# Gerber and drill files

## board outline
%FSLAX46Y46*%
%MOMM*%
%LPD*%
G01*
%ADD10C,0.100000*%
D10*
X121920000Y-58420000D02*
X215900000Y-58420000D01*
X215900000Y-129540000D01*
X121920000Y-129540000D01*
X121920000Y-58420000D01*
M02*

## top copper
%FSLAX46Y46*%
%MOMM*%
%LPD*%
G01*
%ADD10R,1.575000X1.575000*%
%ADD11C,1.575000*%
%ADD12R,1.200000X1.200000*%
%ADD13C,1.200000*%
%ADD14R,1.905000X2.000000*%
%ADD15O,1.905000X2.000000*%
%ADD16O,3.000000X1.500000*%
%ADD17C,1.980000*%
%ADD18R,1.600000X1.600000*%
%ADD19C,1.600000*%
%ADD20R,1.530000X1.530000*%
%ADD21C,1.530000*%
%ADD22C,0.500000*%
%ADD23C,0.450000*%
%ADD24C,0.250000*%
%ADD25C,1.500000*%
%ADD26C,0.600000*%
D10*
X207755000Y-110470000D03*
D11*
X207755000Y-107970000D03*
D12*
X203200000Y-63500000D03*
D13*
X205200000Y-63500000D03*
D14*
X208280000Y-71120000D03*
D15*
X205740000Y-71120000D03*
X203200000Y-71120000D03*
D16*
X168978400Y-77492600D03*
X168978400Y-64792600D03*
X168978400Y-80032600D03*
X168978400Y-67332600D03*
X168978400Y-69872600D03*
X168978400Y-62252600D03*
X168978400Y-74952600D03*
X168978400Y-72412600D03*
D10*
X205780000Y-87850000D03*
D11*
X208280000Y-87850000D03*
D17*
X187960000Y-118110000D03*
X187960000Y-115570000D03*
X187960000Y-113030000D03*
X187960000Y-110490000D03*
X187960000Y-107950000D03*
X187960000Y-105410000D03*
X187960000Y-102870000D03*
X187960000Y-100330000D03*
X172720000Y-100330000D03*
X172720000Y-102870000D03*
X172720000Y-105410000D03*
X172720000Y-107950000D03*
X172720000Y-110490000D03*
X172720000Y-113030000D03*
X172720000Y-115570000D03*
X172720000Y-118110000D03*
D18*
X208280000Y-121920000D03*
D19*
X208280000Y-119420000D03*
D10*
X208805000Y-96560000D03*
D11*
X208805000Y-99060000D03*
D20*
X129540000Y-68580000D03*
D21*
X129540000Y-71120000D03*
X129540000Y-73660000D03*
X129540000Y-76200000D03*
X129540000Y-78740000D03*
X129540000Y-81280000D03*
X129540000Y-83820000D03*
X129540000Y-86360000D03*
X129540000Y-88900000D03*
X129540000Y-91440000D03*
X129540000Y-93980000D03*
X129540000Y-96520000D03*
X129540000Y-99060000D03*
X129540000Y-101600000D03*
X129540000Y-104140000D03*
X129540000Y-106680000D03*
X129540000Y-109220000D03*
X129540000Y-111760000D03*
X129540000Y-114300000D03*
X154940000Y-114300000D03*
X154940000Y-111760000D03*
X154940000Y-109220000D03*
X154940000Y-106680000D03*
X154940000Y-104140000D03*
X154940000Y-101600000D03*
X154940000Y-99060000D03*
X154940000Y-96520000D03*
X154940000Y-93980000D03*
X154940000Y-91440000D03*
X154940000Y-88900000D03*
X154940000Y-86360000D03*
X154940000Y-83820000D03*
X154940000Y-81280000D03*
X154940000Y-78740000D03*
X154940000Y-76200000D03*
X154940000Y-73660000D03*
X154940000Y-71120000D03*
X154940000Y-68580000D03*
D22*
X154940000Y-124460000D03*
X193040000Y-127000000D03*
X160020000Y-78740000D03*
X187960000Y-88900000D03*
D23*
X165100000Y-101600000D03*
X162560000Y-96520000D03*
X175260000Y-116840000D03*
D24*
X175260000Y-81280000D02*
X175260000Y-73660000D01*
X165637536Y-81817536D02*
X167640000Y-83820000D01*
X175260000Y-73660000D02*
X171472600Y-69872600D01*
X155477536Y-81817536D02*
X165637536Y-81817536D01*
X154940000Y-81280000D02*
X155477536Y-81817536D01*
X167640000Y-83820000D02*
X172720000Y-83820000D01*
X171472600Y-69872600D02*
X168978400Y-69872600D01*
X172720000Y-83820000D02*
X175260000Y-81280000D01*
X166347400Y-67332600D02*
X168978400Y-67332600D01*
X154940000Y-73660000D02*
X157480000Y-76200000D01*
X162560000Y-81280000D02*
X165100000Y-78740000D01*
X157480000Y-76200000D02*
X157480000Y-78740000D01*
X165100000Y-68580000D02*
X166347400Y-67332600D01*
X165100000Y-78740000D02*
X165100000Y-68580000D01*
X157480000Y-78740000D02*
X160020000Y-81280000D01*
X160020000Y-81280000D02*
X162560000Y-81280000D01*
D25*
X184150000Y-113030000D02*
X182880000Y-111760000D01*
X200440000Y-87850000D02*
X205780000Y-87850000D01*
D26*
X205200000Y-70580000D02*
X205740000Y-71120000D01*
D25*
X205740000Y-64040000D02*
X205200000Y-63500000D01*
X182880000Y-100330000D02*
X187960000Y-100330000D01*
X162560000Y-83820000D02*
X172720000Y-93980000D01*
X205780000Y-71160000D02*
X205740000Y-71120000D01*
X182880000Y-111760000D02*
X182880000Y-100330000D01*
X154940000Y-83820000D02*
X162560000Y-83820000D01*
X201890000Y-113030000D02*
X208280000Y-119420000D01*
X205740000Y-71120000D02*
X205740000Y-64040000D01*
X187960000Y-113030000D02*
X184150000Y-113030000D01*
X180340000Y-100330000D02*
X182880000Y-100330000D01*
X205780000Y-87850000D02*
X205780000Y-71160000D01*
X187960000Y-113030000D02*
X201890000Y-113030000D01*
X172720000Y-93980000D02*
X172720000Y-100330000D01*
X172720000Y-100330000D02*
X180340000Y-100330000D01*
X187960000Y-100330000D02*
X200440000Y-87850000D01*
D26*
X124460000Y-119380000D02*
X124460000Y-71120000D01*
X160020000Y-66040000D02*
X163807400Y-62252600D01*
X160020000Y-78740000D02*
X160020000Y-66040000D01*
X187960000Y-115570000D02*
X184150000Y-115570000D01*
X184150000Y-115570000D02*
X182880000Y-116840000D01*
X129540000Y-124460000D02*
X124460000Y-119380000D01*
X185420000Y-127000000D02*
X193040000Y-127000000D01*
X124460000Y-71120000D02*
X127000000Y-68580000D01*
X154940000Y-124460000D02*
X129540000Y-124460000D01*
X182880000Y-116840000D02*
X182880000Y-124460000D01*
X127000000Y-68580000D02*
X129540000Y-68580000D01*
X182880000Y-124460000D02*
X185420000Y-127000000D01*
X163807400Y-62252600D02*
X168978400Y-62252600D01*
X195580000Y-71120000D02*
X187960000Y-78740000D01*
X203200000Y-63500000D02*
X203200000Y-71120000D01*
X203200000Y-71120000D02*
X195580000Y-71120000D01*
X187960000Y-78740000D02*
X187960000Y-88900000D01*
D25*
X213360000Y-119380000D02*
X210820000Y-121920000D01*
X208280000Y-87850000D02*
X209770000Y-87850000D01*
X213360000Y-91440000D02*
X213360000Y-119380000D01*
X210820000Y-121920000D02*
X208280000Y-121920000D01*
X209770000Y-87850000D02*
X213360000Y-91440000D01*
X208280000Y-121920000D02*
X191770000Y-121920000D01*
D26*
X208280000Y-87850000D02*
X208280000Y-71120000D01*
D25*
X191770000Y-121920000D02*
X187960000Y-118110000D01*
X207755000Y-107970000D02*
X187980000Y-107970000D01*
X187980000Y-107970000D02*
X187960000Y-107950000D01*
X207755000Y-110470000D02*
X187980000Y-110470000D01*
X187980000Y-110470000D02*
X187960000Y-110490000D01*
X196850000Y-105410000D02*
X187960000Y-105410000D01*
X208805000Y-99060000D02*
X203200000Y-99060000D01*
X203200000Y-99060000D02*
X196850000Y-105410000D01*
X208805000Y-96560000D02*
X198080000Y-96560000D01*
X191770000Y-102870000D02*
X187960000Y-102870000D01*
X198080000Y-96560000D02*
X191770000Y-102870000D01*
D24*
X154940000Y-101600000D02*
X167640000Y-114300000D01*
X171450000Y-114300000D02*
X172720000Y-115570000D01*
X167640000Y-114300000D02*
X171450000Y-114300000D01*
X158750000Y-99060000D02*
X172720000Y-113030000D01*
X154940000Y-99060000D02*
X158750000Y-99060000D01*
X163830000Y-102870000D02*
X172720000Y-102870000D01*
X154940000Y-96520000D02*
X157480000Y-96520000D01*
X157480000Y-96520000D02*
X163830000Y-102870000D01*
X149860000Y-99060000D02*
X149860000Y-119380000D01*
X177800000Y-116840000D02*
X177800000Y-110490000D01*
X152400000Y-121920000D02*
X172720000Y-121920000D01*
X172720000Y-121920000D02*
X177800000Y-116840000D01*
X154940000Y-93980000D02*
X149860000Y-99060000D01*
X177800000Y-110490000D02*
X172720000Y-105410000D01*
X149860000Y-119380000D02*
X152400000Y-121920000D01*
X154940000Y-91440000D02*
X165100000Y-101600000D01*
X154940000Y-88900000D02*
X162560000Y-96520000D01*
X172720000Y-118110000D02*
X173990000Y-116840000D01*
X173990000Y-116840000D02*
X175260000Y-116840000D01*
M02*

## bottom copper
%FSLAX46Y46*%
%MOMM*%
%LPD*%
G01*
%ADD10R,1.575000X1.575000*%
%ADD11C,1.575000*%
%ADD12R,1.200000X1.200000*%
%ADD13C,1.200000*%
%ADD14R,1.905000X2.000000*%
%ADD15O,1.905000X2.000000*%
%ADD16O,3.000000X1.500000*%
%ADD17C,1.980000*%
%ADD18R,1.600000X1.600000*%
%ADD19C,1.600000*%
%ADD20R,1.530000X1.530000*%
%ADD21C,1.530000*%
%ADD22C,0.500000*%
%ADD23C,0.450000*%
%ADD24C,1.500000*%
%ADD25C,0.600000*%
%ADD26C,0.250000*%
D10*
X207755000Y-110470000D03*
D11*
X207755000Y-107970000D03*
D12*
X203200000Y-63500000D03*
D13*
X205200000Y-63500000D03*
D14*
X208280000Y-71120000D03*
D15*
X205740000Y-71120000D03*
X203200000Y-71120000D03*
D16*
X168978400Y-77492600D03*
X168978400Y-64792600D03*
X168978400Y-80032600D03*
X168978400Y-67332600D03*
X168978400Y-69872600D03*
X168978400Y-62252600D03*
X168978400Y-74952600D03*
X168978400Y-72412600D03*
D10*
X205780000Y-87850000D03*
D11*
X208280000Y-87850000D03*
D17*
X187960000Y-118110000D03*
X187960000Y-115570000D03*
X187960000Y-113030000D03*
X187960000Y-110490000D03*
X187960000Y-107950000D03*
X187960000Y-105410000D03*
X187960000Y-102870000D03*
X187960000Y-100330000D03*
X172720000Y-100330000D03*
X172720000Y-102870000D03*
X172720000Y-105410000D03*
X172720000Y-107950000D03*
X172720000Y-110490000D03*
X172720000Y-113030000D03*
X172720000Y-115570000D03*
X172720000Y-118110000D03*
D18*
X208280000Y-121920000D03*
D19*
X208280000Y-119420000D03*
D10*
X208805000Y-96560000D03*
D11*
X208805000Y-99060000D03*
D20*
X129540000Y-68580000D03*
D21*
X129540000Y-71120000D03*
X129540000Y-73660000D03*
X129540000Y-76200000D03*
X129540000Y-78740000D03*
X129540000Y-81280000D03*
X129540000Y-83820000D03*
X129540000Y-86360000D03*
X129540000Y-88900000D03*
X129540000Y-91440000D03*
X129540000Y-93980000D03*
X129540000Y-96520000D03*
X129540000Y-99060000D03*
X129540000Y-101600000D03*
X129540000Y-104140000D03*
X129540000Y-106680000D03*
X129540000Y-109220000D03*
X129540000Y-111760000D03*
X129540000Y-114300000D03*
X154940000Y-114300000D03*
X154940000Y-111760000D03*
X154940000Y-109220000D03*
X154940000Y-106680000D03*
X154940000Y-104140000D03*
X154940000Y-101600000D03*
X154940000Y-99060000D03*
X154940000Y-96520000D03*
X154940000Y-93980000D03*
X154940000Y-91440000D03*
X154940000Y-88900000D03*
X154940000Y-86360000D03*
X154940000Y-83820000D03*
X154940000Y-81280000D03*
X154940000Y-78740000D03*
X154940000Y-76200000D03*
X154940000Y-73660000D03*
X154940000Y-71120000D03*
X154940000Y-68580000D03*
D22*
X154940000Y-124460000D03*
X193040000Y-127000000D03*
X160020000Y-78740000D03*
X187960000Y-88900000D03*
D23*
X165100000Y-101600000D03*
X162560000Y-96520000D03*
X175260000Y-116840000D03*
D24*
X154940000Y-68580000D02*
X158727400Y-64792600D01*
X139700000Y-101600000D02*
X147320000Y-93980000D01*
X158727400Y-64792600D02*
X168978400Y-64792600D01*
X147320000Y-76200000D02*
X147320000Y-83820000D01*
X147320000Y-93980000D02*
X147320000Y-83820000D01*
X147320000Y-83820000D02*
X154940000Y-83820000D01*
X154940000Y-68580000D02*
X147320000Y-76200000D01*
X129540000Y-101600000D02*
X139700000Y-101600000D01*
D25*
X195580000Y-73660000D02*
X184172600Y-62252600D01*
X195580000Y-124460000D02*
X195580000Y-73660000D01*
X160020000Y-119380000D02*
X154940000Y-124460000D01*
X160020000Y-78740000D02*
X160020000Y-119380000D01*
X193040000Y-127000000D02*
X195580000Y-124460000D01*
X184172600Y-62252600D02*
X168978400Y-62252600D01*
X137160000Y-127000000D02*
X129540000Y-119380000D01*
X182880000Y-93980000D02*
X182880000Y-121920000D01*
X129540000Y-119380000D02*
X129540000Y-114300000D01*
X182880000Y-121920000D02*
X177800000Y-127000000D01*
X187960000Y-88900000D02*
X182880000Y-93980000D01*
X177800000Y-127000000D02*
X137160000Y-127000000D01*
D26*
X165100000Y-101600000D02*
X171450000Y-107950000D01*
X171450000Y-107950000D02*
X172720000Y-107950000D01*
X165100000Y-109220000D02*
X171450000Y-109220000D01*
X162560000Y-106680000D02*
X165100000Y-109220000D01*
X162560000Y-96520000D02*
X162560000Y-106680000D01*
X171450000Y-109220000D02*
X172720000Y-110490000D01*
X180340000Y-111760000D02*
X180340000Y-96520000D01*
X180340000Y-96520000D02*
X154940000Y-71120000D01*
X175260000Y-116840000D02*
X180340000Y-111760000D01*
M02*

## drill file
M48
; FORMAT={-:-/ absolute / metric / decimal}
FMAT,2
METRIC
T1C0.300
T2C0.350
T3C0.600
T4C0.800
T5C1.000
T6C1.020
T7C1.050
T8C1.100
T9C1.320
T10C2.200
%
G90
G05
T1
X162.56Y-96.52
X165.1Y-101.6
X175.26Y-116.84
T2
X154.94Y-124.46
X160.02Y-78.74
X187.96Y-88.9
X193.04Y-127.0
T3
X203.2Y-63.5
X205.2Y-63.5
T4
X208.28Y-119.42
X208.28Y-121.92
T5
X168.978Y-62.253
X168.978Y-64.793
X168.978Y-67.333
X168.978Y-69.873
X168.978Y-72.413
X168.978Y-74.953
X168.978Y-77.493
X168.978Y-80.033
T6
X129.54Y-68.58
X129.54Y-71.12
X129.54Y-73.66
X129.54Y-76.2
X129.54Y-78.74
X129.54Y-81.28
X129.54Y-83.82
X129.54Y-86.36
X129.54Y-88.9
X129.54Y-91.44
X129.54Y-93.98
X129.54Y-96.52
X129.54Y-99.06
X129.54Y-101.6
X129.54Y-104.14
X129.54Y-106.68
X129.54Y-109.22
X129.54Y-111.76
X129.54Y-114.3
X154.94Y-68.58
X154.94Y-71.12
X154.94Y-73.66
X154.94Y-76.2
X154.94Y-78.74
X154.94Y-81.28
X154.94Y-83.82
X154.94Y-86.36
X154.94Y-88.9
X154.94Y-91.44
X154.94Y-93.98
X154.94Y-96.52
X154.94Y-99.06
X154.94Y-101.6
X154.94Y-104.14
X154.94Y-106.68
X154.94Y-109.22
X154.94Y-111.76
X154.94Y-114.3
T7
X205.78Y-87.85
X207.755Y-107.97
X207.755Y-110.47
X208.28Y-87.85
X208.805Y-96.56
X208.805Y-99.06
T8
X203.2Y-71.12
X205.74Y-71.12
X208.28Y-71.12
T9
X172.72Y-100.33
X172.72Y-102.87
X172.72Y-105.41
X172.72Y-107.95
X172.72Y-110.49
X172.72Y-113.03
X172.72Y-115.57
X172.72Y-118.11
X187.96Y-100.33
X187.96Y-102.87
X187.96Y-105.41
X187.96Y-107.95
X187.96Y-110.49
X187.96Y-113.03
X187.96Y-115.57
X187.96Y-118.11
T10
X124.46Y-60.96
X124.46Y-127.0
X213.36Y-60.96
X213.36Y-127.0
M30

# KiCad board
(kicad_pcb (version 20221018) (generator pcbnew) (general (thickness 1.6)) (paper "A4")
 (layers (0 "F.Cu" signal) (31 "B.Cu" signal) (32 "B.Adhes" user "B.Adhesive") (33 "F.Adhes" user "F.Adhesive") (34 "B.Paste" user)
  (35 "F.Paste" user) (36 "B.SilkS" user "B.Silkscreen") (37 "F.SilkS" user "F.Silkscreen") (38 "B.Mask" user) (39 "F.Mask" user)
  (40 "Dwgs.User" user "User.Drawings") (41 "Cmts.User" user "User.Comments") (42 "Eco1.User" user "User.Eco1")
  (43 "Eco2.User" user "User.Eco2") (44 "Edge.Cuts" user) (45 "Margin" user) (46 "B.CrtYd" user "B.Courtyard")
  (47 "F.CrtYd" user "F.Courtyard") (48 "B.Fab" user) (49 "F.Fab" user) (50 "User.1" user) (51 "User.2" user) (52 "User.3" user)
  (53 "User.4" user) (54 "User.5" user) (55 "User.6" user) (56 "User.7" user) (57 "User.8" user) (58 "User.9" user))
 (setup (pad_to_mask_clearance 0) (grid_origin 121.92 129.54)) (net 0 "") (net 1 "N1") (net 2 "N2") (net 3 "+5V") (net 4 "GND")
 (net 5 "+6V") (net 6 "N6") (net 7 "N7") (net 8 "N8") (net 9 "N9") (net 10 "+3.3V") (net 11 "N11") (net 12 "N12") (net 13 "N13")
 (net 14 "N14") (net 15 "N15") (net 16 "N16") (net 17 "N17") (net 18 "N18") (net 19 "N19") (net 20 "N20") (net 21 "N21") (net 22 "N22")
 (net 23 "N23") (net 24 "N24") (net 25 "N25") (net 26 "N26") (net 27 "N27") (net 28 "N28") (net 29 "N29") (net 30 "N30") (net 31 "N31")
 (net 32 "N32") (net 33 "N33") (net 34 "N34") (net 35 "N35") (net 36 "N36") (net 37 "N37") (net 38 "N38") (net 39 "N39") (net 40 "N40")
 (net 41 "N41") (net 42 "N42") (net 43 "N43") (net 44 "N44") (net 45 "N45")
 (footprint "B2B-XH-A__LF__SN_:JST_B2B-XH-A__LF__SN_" (layer "F.Cu") (at 208.28 109.22 -90)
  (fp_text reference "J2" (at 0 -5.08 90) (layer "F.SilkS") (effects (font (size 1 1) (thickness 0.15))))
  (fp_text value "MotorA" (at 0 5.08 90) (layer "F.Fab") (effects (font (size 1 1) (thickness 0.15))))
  (pad "1" thru_hole rect (at 1.25 0.525 270) (size 1.575 1.575) (drill 1.05) (layers "*.Cu" "*.Mask") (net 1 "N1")
   (solder_mask_margin 0.102))
  (pad "2" thru_hole circle (at -1.25 0.525 270) (size 1.575 1.575) (drill 1.05) (layers "*.Cu" "*.Mask") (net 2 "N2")
   (solder_mask_margin 0.102)))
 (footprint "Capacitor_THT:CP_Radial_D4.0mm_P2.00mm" (layer "F.Cu") (at 203.2 63.5)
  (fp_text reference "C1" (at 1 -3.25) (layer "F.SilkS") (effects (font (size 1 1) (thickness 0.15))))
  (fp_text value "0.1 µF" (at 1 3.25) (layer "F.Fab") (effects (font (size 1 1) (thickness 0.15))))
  (pad "1" thru_hole rect (at 0 0) (size 1.2 1.2) (drill 0.6) (layers "*.Cu" "*.Mask") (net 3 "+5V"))
  (pad "2" thru_hole circle (at 2 0) (size 1.2 1.2) (drill 0.6) (layers "*.Cu" "*.Mask") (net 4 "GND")))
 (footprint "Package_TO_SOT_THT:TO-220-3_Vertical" (layer "F.Cu") (at 208.28 71.12 180)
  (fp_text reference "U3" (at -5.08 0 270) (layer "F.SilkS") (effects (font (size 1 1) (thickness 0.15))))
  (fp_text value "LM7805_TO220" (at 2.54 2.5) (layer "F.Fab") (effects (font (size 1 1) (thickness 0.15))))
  (pad "1" thru_hole rect (at 0 0 180) (size 1.905 2) (drill 1.1) (layers "*.Cu" "*.Mask") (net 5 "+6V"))
  (pad "2" thru_hole oval (at 2.54 0 180) (size 1.905 2) (drill 1.1) (layers "*.Cu" "*.Mask") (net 4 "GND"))
  (pad "3" thru_hole oval (at 5.08 0 180) (size 1.905 2) (drill 1.1) (layers "*.Cu" "*.Mask") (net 3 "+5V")))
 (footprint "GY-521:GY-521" (layer "F.Cu") (at 167.2084 82.0966)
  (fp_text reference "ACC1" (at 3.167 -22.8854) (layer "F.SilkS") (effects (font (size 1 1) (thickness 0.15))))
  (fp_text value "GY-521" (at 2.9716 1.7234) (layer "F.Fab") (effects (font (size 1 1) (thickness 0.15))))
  (pad "AD0" thru_hole oval (at 1.77 -4.604) (size 3 1.5) (drill 1) (layers "*.Cu" "*.Mask") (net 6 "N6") (solder_mask_margin 0.102))
  (pad "GND" thru_hole oval (at 1.77 -17.304) (size 3 1.5) (drill 1) (layers "*.Cu" "*.Mask") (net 4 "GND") (solder_mask_margin 0.102))
  (pad "INT" thru_hole oval (at 1.77 -2.064) (size 3 1.5) (drill 1) (layers "*.Cu" "*.Mask") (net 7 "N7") (solder_mask_margin 0.102))
  (pad "SCL" thru_hole oval (at 1.77 -14.764) (size 3 1.5) (drill 1) (layers "*.Cu" "*.Mask") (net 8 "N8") (solder_mask_margin 0.102))
  (pad "SDA" thru_hole oval (at 1.77 -12.224) (size 3 1.5) (drill 1) (layers "*.Cu" "*.Mask") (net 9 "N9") (solder_mask_margin 0.102))
  (pad "VCC" thru_hole oval (at 1.77 -19.844) (size 3 1.5) (drill 1) (layers "*.Cu" "*.Mask") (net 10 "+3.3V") (solder_mask_margin 0.102))
  (pad "XCL" thru_hole oval (at 1.77 -7.144) (size 3 1.5) (drill 1) (layers "*.Cu" "*.Mask") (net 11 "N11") (solder_mask_margin 0.102))
  (pad "XDA" thru_hole oval (at 1.77 -9.684) (size 3 1.5) (drill 1) (layers "*.Cu" "*.Mask") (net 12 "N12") (solder_mask_margin 0.102)))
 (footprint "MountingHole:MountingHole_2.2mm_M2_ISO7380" (layer "F.Cu") (at 213.36 127)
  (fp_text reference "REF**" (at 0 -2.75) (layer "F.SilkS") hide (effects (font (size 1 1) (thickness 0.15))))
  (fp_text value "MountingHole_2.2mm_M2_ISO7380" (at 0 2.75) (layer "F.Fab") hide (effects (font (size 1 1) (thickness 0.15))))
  (pad "" np_thru_hole circle (at 0 0) (size 2.2 2.2) (drill 2.2) (layers "F&B.Cu" "*.Mask")))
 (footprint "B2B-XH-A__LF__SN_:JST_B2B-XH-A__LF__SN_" (layer "F.Cu") (at 207.03 88.375 180)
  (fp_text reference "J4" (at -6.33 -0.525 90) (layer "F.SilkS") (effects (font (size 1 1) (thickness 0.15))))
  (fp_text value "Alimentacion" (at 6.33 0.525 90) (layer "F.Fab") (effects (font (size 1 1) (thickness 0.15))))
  (pad "1" thru_hole rect (at 1.25 0.525 180) (size 1.575 1.575) (drill 1.05) (layers "*.Cu" "*.Mask") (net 4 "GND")
   (solder_mask_margin 0.102))
  (pad "2" thru_hole circle (at -1.25 0.525 180) (size 1.575 1.575) (drill 1.05) (layers "*.Cu" "*.Mask") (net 5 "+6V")
   (solder_mask_margin 0.102)))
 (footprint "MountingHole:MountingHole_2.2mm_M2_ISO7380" (layer "F.Cu") (at 213.36 60.96)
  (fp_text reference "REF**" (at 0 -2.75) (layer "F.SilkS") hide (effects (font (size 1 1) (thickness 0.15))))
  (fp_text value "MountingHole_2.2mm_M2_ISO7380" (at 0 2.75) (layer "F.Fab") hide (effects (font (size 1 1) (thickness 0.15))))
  (pad "" np_thru_hole circle (at 0 0) (size 2.2 2.2) (drill 2.2) (layers "F&B.Cu" "*.Mask")))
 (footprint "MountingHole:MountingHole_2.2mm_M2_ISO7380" (layer "F.Cu") (at 124.46 60.96)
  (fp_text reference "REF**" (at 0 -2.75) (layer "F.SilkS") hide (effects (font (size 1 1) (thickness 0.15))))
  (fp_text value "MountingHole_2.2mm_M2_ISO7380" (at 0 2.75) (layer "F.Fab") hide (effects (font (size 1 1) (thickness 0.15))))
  (pad "" np_thru_hole circle (at 0 0) (size 2.2 2.2) (drill 2.2) (layers "F&B.Cu" "*.Mask")))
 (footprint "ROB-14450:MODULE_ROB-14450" (layer "F.Cu") (at 180.34 109.22 180)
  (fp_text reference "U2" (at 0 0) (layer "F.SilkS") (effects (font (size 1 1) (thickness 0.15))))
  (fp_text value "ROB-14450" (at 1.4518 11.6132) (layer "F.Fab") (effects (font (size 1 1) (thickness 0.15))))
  (pad "1" thru_hole circle (at -7.62 -8.89 180) (size 1.98 1.98) (drill 1.32) (layers "*.Cu" "*.Mask") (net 5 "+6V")
   (solder_mask_margin 0.102))
  (pad "2" thru_hole circle (at -7.62 -6.35 180) (size 1.98 1.98) (drill 1.32) (layers "*.Cu" "*.Mask") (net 10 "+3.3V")
   (solder_mask_margin 0.102))
  (pad "3" thru_hole circle (at -7.62 -3.81 180) (size 1.98 1.98) (drill 1.32) (layers "*.Cu" "*.Mask") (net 4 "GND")
   (solder_mask_margin 0.102))
  (pad "4" thru_hole circle (at -7.62 -1.27 180) (size 1.98 1.98) (drill 1.32) (layers "*.Cu" "*.Mask") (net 1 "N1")
   (solder_mask_margin 0.102))
  (pad "5" thru_hole circle (at -7.62 1.27 180) (size 1.98 1.98) (drill 1.32) (layers "*.Cu" "*.Mask") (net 2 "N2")
   (solder_mask_margin 0.102))
  (pad "6" thru_hole circle (at -7.62 3.81 180) (size 1.98 1.98) (drill 1.32) (layers "*.Cu" "*.Mask") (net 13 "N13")
   (solder_mask_margin 0.102))
  (pad "7" thru_hole circle (at -7.62 6.35 180) (size 1.98 1.98) (drill 1.32) (layers "*.Cu" "*.Mask") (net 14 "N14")
   (solder_mask_margin 0.102))
  (pad "8" thru_hole circle (at -7.62 8.89 180) (size 1.98 1.98) (drill 1.32) (layers "*.Cu" "*.Mask") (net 4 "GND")
   (solder_mask_margin 0.102))
  (pad "9" thru_hole circle (at 7.62 8.89 180) (size 1.98 1.98) (drill 1.32) (layers "*.Cu" "*.Mask") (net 4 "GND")
   (solder_mask_margin 0.102))
  (pad "10" thru_hole circle (at 7.62 6.35 180) (size 1.98 1.98) (drill 1.32) (layers "*.Cu" "*.Mask") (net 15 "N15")
   (solder_mask_margin 0.102))
  (pad "11" thru_hole circle (at 7.62 3.81 180) (size 1.98 1.98) (drill 1.32) (layers "*.Cu" "*.Mask") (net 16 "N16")
   (solder_mask_margin 0.102))
  (pad "12" thru_hole circle (at 7.62 1.27 180) (size 1.98 1.98) (drill 1.32) (layers "*.Cu" "*.Mask") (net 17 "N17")
   (solder_mask_margin 0.102))
  (pad "13" thru_hole circle (at 7.62 -1.27 180) (size 1.98 1.98) (drill 1.32) (layers "*.Cu" "*.Mask") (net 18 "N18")
   (solder_mask_margin 0.102))
  (pad "14" thru_hole circle (at 7.62 -3.81 180) (size 1.98 1.98) (drill 1.32) (layers "*.Cu" "*.Mask") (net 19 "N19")
   (solder_mask_margin 0.102))
  (pad "15" thru_hole circle (at 7.62 -6.35 180) (size 1.98 1.98) (drill 1.32) (layers "*.Cu" "*.Mask") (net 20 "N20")
   (solder_mask_margin 0.102))
  (pad "16" thru_hole circle (at 7.62 -8.89 180) (size 1.98 1.98) (drill 1.32) (layers "*.Cu" "*.Mask") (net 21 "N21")
   (solder_mask_margin 0.102)))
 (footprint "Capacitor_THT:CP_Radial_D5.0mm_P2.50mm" (layer "F.Cu") (at 208.28 121.92 90)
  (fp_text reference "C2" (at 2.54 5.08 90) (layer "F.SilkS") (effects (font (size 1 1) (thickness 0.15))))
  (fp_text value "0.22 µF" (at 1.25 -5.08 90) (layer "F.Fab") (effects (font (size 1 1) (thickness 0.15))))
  (pad "1" thru_hole rect (at 0 0 90) (size 1.6 1.6) (drill 0.8) (layers "*.Cu" "*.Mask") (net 5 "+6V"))
  (pad "2" thru_hole circle (at 2.5 0 90) (size 1.6 1.6) (drill 0.8) (layers "*.Cu" "*.Mask") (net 4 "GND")))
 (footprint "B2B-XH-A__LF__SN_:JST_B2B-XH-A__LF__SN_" (layer "F.Cu") (at 208.28 97.81 90)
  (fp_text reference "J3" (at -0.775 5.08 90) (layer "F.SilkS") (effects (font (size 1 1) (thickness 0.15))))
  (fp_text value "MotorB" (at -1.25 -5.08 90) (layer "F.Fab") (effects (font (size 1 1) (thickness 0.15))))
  (pad "1" thru_hole rect (at 1.25 0.525 90) (size 1.575 1.575) (drill 1.05) (layers "*.Cu" "*.Mask") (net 14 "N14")
   (solder_mask_margin 0.102))
  (pad "2" thru_hole circle (at -1.25 0.525 90) (size 1.575 1.575) (drill 1.05) (layers "*.Cu" "*.Mask") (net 13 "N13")
   (solder_mask_margin 0.102)))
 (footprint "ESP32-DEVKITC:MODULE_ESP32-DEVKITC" (layer "F.Cu") (at 142.24 91.43)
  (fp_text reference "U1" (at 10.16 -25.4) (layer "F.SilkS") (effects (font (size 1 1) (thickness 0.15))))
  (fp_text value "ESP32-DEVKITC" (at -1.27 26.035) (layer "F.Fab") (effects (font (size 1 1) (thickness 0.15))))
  (pad "1" thru_hole rect (at -12.7 -22.85) (size 1.53 1.53) (drill 1.02) (layers "*.Cu" "*.Mask") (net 10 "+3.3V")
   (solder_mask_margin 0.102))
  (pad "2" thru_hole circle (at -12.7 -20.31) (size 1.53 1.53) (drill 1.02) (layers "*.Cu" "*.Mask") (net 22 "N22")
   (solder_mask_margin 0.102))
  (pad "3" thru_hole circle (at -12.7 -17.77) (size 1.53 1.53) (drill 1.02) (layers "*.Cu" "*.Mask") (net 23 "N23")
   (solder_mask_margin 0.102))
  (pad "4" thru_hole circle (at -12.7 -15.23) (size 1.53 1.53) (drill 1.02) (layers "*.Cu" "*.Mask") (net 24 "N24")
   (solder_mask_margin 0.102))
  (pad "5" thru_hole circle (at -12.7 -12.69) (size 1.53 1.53) (drill 1.02) (layers "*.Cu" "*.Mask") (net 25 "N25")
   (solder_mask_margin 0.102))
  (pad "6" thru_hole circle (at -12.7 -10.15) (size 1.53 1.53) (drill 1.02) (layers "*.Cu" "*.Mask") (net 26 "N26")
   (solder_mask_margin 0.102))
  (pad "7" thru_hole circle (at -12.7 -7.61) (size 1.53 1.53) (drill 1.02) (layers "*.Cu" "*.Mask") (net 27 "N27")
   (solder_mask_margin 0.102))
  (pad "8" thru_hole circle (at -12.7 -5.07) (size 1.53 1.53) (drill 1.02) (layers "*.Cu" "*.Mask") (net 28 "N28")
   (solder_mask_margin 0.102))
  (pad "9" thru_hole circle (at -12.7 -2.53) (size 1.53 1.53) (drill 1.02) (layers "*.Cu" "*.Mask") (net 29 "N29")
   (solder_mask_margin 0.102))
  (pad "10" thru_hole circle (at -12.7 0.01) (size 1.53 1.53) (drill 1.02) (layers "*.Cu" "*.Mask") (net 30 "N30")
   (solder_mask_margin 0.102))
  (pad "11" thru_hole circle (at -12.7 2.55) (size 1.53 1.53) (drill 1.02) (layers "*.Cu" "*.Mask") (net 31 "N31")
   (solder_mask_margin 0.102))
  (pad "12" thru_hole circle (at -12.7 5.09) (size 1.53 1.53) (drill 1.02) (layers "*.Cu" "*.Mask") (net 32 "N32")
   (solder_mask_margin 0.102))
  (pad "13" thru_hole circle (at -12.7 7.63) (size 1.53 1.53) (drill 1.02) (layers "*.Cu" "*.Mask") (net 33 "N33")
   (solder_mask_margin 0.102))
  (pad "14" thru_hole circle (at -12.7 10.17) (size 1.53 1.53) (drill 1.02) (layers "*.Cu" "*.Mask") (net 4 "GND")
   (solder_mask_margin 0.102))
  (pad "15" thru_hole circle (at -12.7 12.71) (size 1.53 1.53) (drill 1.02) (layers "*.Cu" "*.Mask") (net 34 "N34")
   (solder_mask_margin 0.102))
  (pad "16" thru_hole circle (at -12.7 15.25) (size 1.53 1.53) (drill 1.02) (layers "*.Cu" "*.Mask") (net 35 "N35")
   (solder_mask_margin 0.102))
  (pad "17" thru_hole circle (at -12.7 17.79) (size 1.53 1.53) (drill 1.02) (layers "*.Cu" "*.Mask") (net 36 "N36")
   (solder_mask_margin 0.102))
  (pad "18" thru_hole circle (at -12.7 20.33) (size 1.53 1.53) (drill 1.02) (layers "*.Cu" "*.Mask") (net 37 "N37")
   (solder_mask_margin 0.102))
  (pad "19" thru_hole circle (at -12.7 22.87) (size 1.53 1.53) (drill 1.02) (layers "*.Cu" "*.Mask") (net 3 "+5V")
   (solder_mask_margin 0.102))
  (pad "20" thru_hole circle (at 12.7 22.87) (size 1.53 1.53) (drill 1.02) (layers "*.Cu" "*.Mask") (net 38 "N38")
   (solder_mask_margin 0.102))
  (pad "21" thru_hole circle (at 12.7 20.33) (size 1.53 1.53) (drill 1.02) (layers "*.Cu" "*.Mask") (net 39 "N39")
   (solder_mask_margin 0.102))
  (pad "22" thru_hole circle (at 12.7 17.79) (size 1.53 1.53) (drill 1.02) (layers "*.Cu" "*.Mask") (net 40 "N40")
   (solder_mask_margin 0.102))
  (pad "23" thru_hole circle (at 12.7 15.25) (size 1.53 1.53) (drill 1.02) (layers "*.Cu" "*.Mask") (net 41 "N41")
   (solder_mask_margin 0.102))
  (pad "24" thru_hole circle (at 12.7 12.71) (size 1.53 1.53) (drill 1.02) (layers "*.Cu" "*.Mask") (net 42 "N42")
   (solder_mask_margin 0.102))
  (pad "25" thru_hole circle (at 12.7 10.17) (size 1.53 1.53) (drill 1.02) (layers "*.Cu" "*.Mask") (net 20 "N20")
   (solder_mask_margin 0.102))
  (pad "26" thru_hole circle (at 12.7 7.63) (size 1.53 1.53) (drill 1.02) (layers "*.Cu" "*.Mask") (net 19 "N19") (solder_mask_margin 0.102))
  (pad "27" thru_hole circle (at 12.7 5.09) (size 1.53 1.53) (drill 1.02) (layers "*.Cu" "*.Mask") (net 15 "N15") (solder_mask_margin 0.102))
  (pad "28" thru_hole circle (at 12.7 2.55) (size 1.53 1.53) (drill 1.02) (layers "*.Cu" "*.Mask") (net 16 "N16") (solder_mask_margin 0.102))
  (pad "29" thru_hole circle (at 12.7 0.01) (size 1.53 1.53) (drill 1.02) (layers "*.Cu" "*.Mask") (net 17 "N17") (solder_mask_margin 0.102))
  (pad "30" thru_hole circle (at 12.7 -2.53) (size 1.53 1.53) (drill 1.02) (layers "*.Cu" "*.Mask") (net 18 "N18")
   (solder_mask_margin 0.102))
  (pad "31" thru_hole circle (at 12.7 -5.07) (size 1.53 1.53) (drill 1.02) (layers "*.Cu" "*.Mask") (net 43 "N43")
   (solder_mask_margin 0.102))
  (pad "32" thru_hole circle (at 12.7 -7.61) (size 1.53 1.53) (drill 1.02) (layers "*.Cu" "*.Mask") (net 4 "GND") (solder_mask_margin 0.102))
  (pad "33" thru_hole circle (at 12.7 -10.15) (size 1.53 1.53) (drill 1.02) (layers "*.Cu" "*.Mask") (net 9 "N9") (solder_mask_margin 0.102))
  (pad "34" thru_hole circle (at 12.7 -12.69) (size 1.53 1.53) (drill 1.02) (layers "*.Cu" "*.Mask") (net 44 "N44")
   (solder_mask_margin 0.102))
  (pad "35" thru_hole circle (at 12.7 -15.23) (size 1.53 1.53) (drill 1.02) (layers "*.Cu" "*.Mask") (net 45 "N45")
   (solder_mask_margin 0.102))
  (pad "36" thru_hole circle (at 12.7 -17.77) (size 1.53 1.53) (drill 1.02) (layers "*.Cu" "*.Mask") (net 8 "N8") (solder_mask_margin 0.102))
  (pad "37" thru_hole circle (at 12.7 -20.31) (size 1.53 1.53) (drill 1.02) (layers "*.Cu" "*.Mask") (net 21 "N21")
   (solder_mask_margin 0.102))
  (pad "38" thru_hole circle (at 12.7 -22.85) (size 1.53 1.53) (drill 1.02) (layers "*.Cu" "*.Mask") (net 4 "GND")
   (solder_mask_margin 0.102)))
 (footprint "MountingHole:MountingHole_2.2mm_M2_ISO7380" (layer "F.Cu") (at 124.46 127)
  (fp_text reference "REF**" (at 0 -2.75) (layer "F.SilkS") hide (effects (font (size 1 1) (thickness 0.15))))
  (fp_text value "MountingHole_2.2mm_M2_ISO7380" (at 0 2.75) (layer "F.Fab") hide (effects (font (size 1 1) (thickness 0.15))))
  (pad "" np_thru_hole circle (at 0 0) (size 2.2 2.2) (drill 2.2) (layers "F&B.Cu" "*.Mask")))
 (gr_rect (start 121.92 58.42) (end 215.9 129.54) (stroke (width 0.1) (type default)) (fill none) (layer "Edge.Cuts"))
 (segment (start 175.26 81.28) (end 175.26 73.66) (width 0.25) (layer "F.Cu") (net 9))
 (segment (start 165.637536 81.817536) (end 167.64 83.82) (width 0.25) (layer "F.Cu") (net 9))
 (segment (start 175.26 73.66) (end 171.4726 69.8726) (width 0.25) (layer "F.Cu") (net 9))
 (segment (start 155.477536 81.817536) (end 165.637536 81.817536) (width 0.25) (layer "F.Cu") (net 9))
 (segment (start 154.94 81.28) (end 155.477536 81.817536) (width 0.25) (layer "F.Cu") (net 9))
 (segment (start 167.64 83.82) (end 172.72 83.82) (width 0.25) (layer "F.Cu") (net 9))
 (segment (start 171.4726 69.8726) (end 168.9784 69.8726) (width 0.25) (layer "F.Cu") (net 9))
 (segment (start 172.72 83.82) (end 175.26 81.28) (width 0.25) (layer "F.Cu") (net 9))
 (segment (start 166.3474 67.3326) (end 168.9784 67.3326) (width 0.25) (layer "F.Cu") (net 8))
 (segment (start 154.94 73.66) (end 157.48 76.2) (width 0.25) (layer "F.Cu") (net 8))
 (segment (start 162.56 81.28) (end 165.1 78.74) (width 0.25) (layer "F.Cu") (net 8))
 (segment (start 157.48 76.2) (end 157.48 78.74) (width 0.25) (layer "F.Cu") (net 8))
 (segment (start 165.1 68.58) (end 166.3474 67.3326) (width 0.25) (layer "F.Cu") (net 8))
 (segment (start 165.1 78.74) (end 165.1 68.58) (width 0.25) (layer "F.Cu") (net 8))
 (segment (start 157.48 78.74) (end 160.02 81.28) (width 0.25) (layer "F.Cu") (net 8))
 (segment (start 160.02 81.28) (end 162.56 81.28) (width 0.25) (layer "F.Cu") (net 8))
 (segment (start 184.15 113.03) (end 182.88 111.76) (width 1.5) (layer "F.Cu") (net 4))
 (segment (start 200.44 87.85) (end 205.78 87.85) (width 1.5) (layer "F.Cu") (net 4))
 (segment (start 205.2 70.58) (end 205.74 71.12) (width 0.6) (layer "F.Cu") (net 4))
 (segment (start 205.74 64.04) (end 205.2 63.5) (width 1.5) (layer "F.Cu") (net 4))
 (segment (start 182.88 100.33) (end 187.96 100.33) (width 1.5) (layer "F.Cu") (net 4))
 (segment (start 162.56 83.82) (end 172.72 93.98) (width 1.5) (layer "F.Cu") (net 4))
 (segment (start 205.78 71.16) (end 205.74 71.12) (width 1.5) (layer "F.Cu") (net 4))
 (segment (start 182.88 111.76) (end 182.88 100.33) (width 1.5) (layer "F.Cu") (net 4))
 (segment (start 154.94 83.82) (end 162.56 83.82) (width 1.5) (layer "F.Cu") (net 4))
 (segment (start 201.89 113.03) (end 208.28 119.42) (width 1.5) (layer "F.Cu") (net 4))
 (segment (start 205.74 71.12) (end 205.74 64.04) (width 1.5) (layer "F.Cu") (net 4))
 (segment (start 187.96 113.03) (end 184.15 113.03) (width 1.5) (layer "F.Cu") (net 4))
 (segment (start 180.34 100.33) (end 182.88 100.33) (width 1.5) (layer "F.Cu") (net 4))
 (segment (start 205.78 87.85) (end 205.78 71.16) (width 1.5) (layer "F.Cu") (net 4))
 (segment (start 187.96 113.03) (end 201.89 113.03) (width 1.5) (layer "F.Cu") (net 4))
 (segment (start 172.72 93.98) (end 172.72 100.33) (width 1.5) (layer "F.Cu") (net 4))
 (segment (start 172.72 100.33) (end 180.34 100.33) (width 1.5) (layer "F.Cu") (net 4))
 (segment (start 187.96 100.33) (end 200.44 87.85) (width 1.5) (layer "F.Cu") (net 4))
 (segment (start 154.94 68.58) (end 158.7274 64.7926) (width 1.5) (layer "B.Cu") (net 4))
 (segment (start 139.7 101.6) (end 147.32 93.98) (width 1.5) (layer "B.Cu") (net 4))
 (segment (start 158.7274 64.7926) (end 168.9784 64.7926) (width 1.5) (layer "B.Cu") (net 4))
 (segment (start 147.32 76.2) (end 147.32 83.82) (width 1.5) (layer "B.Cu") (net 4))
 (segment (start 147.32 93.98) (end 147.32 83.82) (width 1.5) (layer "B.Cu") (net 4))
 (segment (start 147.32 83.82) (end 154.94 83.82) (width 1.5) (layer "B.Cu") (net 4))
 (segment (start 154.94 68.58) (end 147.32 76.2) (width 1.5) (layer "B.Cu") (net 4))
 (segment (start 129.54 101.6) (end 139.7 101.6) (width 1.5) (layer "B.Cu") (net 4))
 (segment (start 124.46 119.38) (end 124.46 71.12) (width 0.6) (layer "F.Cu") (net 10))
 (segment (start 160.02 66.04) (end 163.8074 62.2526) (width 0.6) (layer "F.Cu") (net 10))
 (segment (start 160.02 78.74) (end 160.02 66.04) (width 0.6) (layer "F.Cu") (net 10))
 (segment (start 187.96 115.57) (end 184.15 115.57) (width 0.6) (layer "F.Cu") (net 10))
 (segment (start 184.15 115.57) (end 182.88 116.84) (width 0.6) (layer "F.Cu") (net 10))
 (segment (start 129.54 124.46) (end 124.46 119.38) (width 0.6) (layer "F.Cu") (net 10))
 (segment (start 185.42 127) (end 193.04 127) (width 0.6) (layer "F.Cu") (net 10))
 (segment (start 124.46 71.12) (end 127 68.58) (width 0.6) (layer "F.Cu") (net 10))
 (segment (start 154.94 124.46) (end 129.54 124.46) (width 0.6) (layer "F.Cu") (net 10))
 (segment (start 182.88 116.84) (end 182.88 124.46) (width 0.6) (layer "F.Cu") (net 10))
 (segment (start 127 68.58) (end 129.54 68.58) (width 0.6) (layer "F.Cu") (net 10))
 (segment (start 182.88 124.46) (end 185.42 127) (width 0.6) (layer "F.Cu") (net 10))
 (segment (start 163.8074 62.2526) (end 168.9784 62.2526) (width 0.6) (layer "F.Cu") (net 10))
 (via (at 154.94 124.46) (size 0.5) (drill 0.35) (layers "F.Cu" "B.Cu") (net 10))
 (via (at 193.04 127) (size 0.5) (drill 0.35) (layers "F.Cu" "B.Cu") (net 10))
 (via (at 160.02 78.74) (size 0.5) (drill 0.35) (layers "F.Cu" "B.Cu") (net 10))
 (segment (start 195.58 73.66) (end 184.1726 62.2526) (width 0.6) (layer "B.Cu") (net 10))
 (segment (start 195.58 124.46) (end 195.58 73.66) (width 0.6) (layer "B.Cu") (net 10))
 (segment (start 160.02 119.38) (end 154.94 124.46) (width 0.6) (layer "B.Cu") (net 10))
 (segment (start 160.02 78.74) (end 160.02 119.38) (width 0.6) (layer "B.Cu") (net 10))
 (segment (start 193.04 127) (end 195.58 124.46) (width 0.6) (layer "B.Cu") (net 10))
 (segment (start 184.1726 62.2526) (end 168.9784 62.2526) (width 0.6) (layer "B.Cu") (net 10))
 (segment (start 195.58 71.12) (end 187.96 78.74) (width 0.6) (layer "F.Cu") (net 3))
 (segment (start 203.2 63.5) (end 203.2 71.12) (width 0.6) (layer "F.Cu") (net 3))
 (segment (start 203.2 71.12) (end 195.58 71.12) (width 0.6) (layer "F.Cu") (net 3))
 (segment (start 187.96 78.74) (end 187.96 88.9) (width 0.6) (layer "F.Cu") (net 3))
 (via (at 187.96 88.9) (size 0.5) (drill 0.35) (layers "F.Cu" "B.Cu") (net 3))
 (segment (start 137.16 127) (end 129.54 119.38) (width 0.6) (layer "B.Cu") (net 3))
 (segment (start 182.88 93.98) (end 182.88 121.92) (width 0.6) (layer "B.Cu") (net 3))
 (segment (start 129.54 119.38) (end 129.54 114.3) (width 0.6) (layer "B.Cu") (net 3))
 (segment (start 182.88 121.92) (end 177.8 127) (width 0.6) (layer "B.Cu") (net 3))
 (segment (start 187.96 88.9) (end 182.88 93.98) (width 0.6) (layer "B.Cu") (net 3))
 (segment (start 177.8 127) (end 137.16 127) (width 0.6) (layer "B.Cu") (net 3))
 (segment (start 213.36 119.38) (end 210.82 121.92) (width 1.5) (layer "F.Cu") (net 5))
 (segment (start 208.28 87.85) (end 209.77 87.85) (width 1.5) (layer "F.Cu") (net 5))
 (segment (start 213.36 91.44) (end 213.36 119.38) (width 1.5) (layer "F.Cu") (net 5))
 (segment (start 210.82 121.92) (end 208.28 121.92) (width 1.5) (layer "F.Cu") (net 5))
 (segment (start 209.77 87.85) (end 213.36 91.44) (width 1.5) (layer "F.Cu") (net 5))
 (segment (start 208.28 121.92) (end 191.77 121.92) (width 1.5) (layer "F.Cu") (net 5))
 (segment (start 208.28 87.85) (end 208.28 71.12) (width 0.6) (layer "F.Cu") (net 5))
 (segment (start 191.77 121.92) (end 187.96 118.11) (width 1.5) (layer "F.Cu") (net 5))
 (segment (start 207.755 107.97) (end 187.98 107.97) (width 1.5) (layer "F.Cu") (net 2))
 (segment (start 187.98 107.97) (end 187.96 107.95) (width 1.5) (layer "F.Cu") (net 2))
 (segment (start 207.755 110.47) (end 187.98 110.47) (width 1.5) (layer "F.Cu") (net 1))
 (segment (start 187.98 110.47) (end 187.96 110.49) (width 1.5) (layer "F.Cu") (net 1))
 (segment (start 196.85 105.41) (end 187.96 105.41) (width 1.5) (layer "F.Cu") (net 13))
 (segment (start 208.805 99.06) (end 203.2 99.06) (width 1.5) (layer "F.Cu") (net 13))
 (segment (start 203.2 99.06) (end 196.85 105.41) (width 1.5) (layer "F.Cu") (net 13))
 (segment (start 208.805 96.56) (end 198.08 96.56) (width 1.5) (layer "F.Cu") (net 14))
 (segment (start 191.77 102.87) (end 187.96 102.87) (width 1.5) (layer "F.Cu") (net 14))
 (segment (start 198.08 96.56) (end 191.77 102.87) (width 1.5) (layer "F.Cu") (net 14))
 (segment (start 154.94 101.6) (end 167.64 114.3) (width 0.25) (layer "F.Cu") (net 20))
 (segment (start 171.45 114.3) (end 172.72 115.57) (width 0.25) (layer "F.Cu") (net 20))
 (segment (start 167.64 114.3) (end 171.45 114.3) (width 0.25) (layer "F.Cu") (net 20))
 (segment (start 158.75 99.06) (end 172.72 113.03) (width 0.25) (layer "F.Cu") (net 19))
 (segment (start 154.94 99.06) (end 158.75 99.06) (width 0.25) (layer "F.Cu") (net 19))
 (segment (start 163.83 102.87) (end 172.72 102.87) (width 0.25) (layer "F.Cu") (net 15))
 (segment (start 154.94 96.52) (end 157.48 96.52) (width 0.25) (layer "F.Cu") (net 15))
 (segment (start 157.48 96.52) (end 163.83 102.87) (width 0.25) (layer "F.Cu") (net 15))
 (segment (start 149.86 99.06) (end 149.86 119.38) (width 0.25) (layer "F.Cu") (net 16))
 (segment (start 177.8 116.84) (end 177.8 110.49) (width 0.25) (layer "F.Cu") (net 16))
 (segment (start 152.4 121.92) (end 172.72 121.92) (width 0.25) (layer "F.Cu") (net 16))
 (segment (start 172.72 121.92) (end 177.8 116.84) (width 0.25) (layer "F.Cu") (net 16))
 (segment (start 154.94 93.98) (end 149.86 99.06) (width 0.25) (layer "F.Cu") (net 16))
 (segment (start 177.8 110.49) (end 172.72 105.41) (width 0.25) (layer "F.Cu") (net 16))
 (segment (start 149.86 119.38) (end 152.4 121.92) (width 0.25) (layer "F.Cu") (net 16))
 (segment (start 154.94 91.44) (end 165.1 101.6) (width 0.25) (layer "F.Cu") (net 17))
 (via (at 165.1 101.6) (size 0.45) (drill 0.3) (layers "F.Cu" "B.Cu") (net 17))
 (segment (start 165.1 101.6) (end 171.45 107.95) (width 0.25) (layer "B.Cu") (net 17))
 (segment (start 171.45 107.95) (end 172.72 107.95) (width 0.25) (layer "B.Cu") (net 17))
 (segment (start 154.94 88.9) (end 162.56 96.52) (width 0.25) (layer "F.Cu") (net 18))
 (via (at 162.56 96.52) (size 0.45) (drill 0.3) (layers "F.Cu" "B.Cu") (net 18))
 (segment (start 165.1 109.22) (end 171.45 109.22) (width 0.25) (layer "B.Cu") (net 18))
 (segment (start 162.56 106.68) (end 165.1 109.22) (width 0.25) (layer "B.Cu") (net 18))
 (segment (start 162.56 96.52) (end 162.56 106.68) (width 0.25) (layer "B.Cu") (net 18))
 (segment (start 171.45 109.22) (end 172.72 110.49) (width 0.25) (layer "B.Cu") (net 18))
 (segment (start 172.72 118.11) (end 173.99 116.84) (width 0.25) (layer "F.Cu") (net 21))
 (segment (start 173.99 116.84) (end 175.26 116.84) (width 0.25) (layer "F.Cu") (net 21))
 (via (at 175.26 116.84) (size 0.45) (drill 0.3) (layers "F.Cu" "B.Cu") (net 21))
 (segment (start 180.34 111.76) (end 180.34 96.52) (width 0.25) (layer "B.Cu") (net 21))
 (segment (start 180.34 96.52) (end 154.94 71.12) (width 0.25) (layer "B.Cu") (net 21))
 (segment (start 175.26 116.84) (end 180.34 111.76) (width 0.25) (layer "B.Cu") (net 21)))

